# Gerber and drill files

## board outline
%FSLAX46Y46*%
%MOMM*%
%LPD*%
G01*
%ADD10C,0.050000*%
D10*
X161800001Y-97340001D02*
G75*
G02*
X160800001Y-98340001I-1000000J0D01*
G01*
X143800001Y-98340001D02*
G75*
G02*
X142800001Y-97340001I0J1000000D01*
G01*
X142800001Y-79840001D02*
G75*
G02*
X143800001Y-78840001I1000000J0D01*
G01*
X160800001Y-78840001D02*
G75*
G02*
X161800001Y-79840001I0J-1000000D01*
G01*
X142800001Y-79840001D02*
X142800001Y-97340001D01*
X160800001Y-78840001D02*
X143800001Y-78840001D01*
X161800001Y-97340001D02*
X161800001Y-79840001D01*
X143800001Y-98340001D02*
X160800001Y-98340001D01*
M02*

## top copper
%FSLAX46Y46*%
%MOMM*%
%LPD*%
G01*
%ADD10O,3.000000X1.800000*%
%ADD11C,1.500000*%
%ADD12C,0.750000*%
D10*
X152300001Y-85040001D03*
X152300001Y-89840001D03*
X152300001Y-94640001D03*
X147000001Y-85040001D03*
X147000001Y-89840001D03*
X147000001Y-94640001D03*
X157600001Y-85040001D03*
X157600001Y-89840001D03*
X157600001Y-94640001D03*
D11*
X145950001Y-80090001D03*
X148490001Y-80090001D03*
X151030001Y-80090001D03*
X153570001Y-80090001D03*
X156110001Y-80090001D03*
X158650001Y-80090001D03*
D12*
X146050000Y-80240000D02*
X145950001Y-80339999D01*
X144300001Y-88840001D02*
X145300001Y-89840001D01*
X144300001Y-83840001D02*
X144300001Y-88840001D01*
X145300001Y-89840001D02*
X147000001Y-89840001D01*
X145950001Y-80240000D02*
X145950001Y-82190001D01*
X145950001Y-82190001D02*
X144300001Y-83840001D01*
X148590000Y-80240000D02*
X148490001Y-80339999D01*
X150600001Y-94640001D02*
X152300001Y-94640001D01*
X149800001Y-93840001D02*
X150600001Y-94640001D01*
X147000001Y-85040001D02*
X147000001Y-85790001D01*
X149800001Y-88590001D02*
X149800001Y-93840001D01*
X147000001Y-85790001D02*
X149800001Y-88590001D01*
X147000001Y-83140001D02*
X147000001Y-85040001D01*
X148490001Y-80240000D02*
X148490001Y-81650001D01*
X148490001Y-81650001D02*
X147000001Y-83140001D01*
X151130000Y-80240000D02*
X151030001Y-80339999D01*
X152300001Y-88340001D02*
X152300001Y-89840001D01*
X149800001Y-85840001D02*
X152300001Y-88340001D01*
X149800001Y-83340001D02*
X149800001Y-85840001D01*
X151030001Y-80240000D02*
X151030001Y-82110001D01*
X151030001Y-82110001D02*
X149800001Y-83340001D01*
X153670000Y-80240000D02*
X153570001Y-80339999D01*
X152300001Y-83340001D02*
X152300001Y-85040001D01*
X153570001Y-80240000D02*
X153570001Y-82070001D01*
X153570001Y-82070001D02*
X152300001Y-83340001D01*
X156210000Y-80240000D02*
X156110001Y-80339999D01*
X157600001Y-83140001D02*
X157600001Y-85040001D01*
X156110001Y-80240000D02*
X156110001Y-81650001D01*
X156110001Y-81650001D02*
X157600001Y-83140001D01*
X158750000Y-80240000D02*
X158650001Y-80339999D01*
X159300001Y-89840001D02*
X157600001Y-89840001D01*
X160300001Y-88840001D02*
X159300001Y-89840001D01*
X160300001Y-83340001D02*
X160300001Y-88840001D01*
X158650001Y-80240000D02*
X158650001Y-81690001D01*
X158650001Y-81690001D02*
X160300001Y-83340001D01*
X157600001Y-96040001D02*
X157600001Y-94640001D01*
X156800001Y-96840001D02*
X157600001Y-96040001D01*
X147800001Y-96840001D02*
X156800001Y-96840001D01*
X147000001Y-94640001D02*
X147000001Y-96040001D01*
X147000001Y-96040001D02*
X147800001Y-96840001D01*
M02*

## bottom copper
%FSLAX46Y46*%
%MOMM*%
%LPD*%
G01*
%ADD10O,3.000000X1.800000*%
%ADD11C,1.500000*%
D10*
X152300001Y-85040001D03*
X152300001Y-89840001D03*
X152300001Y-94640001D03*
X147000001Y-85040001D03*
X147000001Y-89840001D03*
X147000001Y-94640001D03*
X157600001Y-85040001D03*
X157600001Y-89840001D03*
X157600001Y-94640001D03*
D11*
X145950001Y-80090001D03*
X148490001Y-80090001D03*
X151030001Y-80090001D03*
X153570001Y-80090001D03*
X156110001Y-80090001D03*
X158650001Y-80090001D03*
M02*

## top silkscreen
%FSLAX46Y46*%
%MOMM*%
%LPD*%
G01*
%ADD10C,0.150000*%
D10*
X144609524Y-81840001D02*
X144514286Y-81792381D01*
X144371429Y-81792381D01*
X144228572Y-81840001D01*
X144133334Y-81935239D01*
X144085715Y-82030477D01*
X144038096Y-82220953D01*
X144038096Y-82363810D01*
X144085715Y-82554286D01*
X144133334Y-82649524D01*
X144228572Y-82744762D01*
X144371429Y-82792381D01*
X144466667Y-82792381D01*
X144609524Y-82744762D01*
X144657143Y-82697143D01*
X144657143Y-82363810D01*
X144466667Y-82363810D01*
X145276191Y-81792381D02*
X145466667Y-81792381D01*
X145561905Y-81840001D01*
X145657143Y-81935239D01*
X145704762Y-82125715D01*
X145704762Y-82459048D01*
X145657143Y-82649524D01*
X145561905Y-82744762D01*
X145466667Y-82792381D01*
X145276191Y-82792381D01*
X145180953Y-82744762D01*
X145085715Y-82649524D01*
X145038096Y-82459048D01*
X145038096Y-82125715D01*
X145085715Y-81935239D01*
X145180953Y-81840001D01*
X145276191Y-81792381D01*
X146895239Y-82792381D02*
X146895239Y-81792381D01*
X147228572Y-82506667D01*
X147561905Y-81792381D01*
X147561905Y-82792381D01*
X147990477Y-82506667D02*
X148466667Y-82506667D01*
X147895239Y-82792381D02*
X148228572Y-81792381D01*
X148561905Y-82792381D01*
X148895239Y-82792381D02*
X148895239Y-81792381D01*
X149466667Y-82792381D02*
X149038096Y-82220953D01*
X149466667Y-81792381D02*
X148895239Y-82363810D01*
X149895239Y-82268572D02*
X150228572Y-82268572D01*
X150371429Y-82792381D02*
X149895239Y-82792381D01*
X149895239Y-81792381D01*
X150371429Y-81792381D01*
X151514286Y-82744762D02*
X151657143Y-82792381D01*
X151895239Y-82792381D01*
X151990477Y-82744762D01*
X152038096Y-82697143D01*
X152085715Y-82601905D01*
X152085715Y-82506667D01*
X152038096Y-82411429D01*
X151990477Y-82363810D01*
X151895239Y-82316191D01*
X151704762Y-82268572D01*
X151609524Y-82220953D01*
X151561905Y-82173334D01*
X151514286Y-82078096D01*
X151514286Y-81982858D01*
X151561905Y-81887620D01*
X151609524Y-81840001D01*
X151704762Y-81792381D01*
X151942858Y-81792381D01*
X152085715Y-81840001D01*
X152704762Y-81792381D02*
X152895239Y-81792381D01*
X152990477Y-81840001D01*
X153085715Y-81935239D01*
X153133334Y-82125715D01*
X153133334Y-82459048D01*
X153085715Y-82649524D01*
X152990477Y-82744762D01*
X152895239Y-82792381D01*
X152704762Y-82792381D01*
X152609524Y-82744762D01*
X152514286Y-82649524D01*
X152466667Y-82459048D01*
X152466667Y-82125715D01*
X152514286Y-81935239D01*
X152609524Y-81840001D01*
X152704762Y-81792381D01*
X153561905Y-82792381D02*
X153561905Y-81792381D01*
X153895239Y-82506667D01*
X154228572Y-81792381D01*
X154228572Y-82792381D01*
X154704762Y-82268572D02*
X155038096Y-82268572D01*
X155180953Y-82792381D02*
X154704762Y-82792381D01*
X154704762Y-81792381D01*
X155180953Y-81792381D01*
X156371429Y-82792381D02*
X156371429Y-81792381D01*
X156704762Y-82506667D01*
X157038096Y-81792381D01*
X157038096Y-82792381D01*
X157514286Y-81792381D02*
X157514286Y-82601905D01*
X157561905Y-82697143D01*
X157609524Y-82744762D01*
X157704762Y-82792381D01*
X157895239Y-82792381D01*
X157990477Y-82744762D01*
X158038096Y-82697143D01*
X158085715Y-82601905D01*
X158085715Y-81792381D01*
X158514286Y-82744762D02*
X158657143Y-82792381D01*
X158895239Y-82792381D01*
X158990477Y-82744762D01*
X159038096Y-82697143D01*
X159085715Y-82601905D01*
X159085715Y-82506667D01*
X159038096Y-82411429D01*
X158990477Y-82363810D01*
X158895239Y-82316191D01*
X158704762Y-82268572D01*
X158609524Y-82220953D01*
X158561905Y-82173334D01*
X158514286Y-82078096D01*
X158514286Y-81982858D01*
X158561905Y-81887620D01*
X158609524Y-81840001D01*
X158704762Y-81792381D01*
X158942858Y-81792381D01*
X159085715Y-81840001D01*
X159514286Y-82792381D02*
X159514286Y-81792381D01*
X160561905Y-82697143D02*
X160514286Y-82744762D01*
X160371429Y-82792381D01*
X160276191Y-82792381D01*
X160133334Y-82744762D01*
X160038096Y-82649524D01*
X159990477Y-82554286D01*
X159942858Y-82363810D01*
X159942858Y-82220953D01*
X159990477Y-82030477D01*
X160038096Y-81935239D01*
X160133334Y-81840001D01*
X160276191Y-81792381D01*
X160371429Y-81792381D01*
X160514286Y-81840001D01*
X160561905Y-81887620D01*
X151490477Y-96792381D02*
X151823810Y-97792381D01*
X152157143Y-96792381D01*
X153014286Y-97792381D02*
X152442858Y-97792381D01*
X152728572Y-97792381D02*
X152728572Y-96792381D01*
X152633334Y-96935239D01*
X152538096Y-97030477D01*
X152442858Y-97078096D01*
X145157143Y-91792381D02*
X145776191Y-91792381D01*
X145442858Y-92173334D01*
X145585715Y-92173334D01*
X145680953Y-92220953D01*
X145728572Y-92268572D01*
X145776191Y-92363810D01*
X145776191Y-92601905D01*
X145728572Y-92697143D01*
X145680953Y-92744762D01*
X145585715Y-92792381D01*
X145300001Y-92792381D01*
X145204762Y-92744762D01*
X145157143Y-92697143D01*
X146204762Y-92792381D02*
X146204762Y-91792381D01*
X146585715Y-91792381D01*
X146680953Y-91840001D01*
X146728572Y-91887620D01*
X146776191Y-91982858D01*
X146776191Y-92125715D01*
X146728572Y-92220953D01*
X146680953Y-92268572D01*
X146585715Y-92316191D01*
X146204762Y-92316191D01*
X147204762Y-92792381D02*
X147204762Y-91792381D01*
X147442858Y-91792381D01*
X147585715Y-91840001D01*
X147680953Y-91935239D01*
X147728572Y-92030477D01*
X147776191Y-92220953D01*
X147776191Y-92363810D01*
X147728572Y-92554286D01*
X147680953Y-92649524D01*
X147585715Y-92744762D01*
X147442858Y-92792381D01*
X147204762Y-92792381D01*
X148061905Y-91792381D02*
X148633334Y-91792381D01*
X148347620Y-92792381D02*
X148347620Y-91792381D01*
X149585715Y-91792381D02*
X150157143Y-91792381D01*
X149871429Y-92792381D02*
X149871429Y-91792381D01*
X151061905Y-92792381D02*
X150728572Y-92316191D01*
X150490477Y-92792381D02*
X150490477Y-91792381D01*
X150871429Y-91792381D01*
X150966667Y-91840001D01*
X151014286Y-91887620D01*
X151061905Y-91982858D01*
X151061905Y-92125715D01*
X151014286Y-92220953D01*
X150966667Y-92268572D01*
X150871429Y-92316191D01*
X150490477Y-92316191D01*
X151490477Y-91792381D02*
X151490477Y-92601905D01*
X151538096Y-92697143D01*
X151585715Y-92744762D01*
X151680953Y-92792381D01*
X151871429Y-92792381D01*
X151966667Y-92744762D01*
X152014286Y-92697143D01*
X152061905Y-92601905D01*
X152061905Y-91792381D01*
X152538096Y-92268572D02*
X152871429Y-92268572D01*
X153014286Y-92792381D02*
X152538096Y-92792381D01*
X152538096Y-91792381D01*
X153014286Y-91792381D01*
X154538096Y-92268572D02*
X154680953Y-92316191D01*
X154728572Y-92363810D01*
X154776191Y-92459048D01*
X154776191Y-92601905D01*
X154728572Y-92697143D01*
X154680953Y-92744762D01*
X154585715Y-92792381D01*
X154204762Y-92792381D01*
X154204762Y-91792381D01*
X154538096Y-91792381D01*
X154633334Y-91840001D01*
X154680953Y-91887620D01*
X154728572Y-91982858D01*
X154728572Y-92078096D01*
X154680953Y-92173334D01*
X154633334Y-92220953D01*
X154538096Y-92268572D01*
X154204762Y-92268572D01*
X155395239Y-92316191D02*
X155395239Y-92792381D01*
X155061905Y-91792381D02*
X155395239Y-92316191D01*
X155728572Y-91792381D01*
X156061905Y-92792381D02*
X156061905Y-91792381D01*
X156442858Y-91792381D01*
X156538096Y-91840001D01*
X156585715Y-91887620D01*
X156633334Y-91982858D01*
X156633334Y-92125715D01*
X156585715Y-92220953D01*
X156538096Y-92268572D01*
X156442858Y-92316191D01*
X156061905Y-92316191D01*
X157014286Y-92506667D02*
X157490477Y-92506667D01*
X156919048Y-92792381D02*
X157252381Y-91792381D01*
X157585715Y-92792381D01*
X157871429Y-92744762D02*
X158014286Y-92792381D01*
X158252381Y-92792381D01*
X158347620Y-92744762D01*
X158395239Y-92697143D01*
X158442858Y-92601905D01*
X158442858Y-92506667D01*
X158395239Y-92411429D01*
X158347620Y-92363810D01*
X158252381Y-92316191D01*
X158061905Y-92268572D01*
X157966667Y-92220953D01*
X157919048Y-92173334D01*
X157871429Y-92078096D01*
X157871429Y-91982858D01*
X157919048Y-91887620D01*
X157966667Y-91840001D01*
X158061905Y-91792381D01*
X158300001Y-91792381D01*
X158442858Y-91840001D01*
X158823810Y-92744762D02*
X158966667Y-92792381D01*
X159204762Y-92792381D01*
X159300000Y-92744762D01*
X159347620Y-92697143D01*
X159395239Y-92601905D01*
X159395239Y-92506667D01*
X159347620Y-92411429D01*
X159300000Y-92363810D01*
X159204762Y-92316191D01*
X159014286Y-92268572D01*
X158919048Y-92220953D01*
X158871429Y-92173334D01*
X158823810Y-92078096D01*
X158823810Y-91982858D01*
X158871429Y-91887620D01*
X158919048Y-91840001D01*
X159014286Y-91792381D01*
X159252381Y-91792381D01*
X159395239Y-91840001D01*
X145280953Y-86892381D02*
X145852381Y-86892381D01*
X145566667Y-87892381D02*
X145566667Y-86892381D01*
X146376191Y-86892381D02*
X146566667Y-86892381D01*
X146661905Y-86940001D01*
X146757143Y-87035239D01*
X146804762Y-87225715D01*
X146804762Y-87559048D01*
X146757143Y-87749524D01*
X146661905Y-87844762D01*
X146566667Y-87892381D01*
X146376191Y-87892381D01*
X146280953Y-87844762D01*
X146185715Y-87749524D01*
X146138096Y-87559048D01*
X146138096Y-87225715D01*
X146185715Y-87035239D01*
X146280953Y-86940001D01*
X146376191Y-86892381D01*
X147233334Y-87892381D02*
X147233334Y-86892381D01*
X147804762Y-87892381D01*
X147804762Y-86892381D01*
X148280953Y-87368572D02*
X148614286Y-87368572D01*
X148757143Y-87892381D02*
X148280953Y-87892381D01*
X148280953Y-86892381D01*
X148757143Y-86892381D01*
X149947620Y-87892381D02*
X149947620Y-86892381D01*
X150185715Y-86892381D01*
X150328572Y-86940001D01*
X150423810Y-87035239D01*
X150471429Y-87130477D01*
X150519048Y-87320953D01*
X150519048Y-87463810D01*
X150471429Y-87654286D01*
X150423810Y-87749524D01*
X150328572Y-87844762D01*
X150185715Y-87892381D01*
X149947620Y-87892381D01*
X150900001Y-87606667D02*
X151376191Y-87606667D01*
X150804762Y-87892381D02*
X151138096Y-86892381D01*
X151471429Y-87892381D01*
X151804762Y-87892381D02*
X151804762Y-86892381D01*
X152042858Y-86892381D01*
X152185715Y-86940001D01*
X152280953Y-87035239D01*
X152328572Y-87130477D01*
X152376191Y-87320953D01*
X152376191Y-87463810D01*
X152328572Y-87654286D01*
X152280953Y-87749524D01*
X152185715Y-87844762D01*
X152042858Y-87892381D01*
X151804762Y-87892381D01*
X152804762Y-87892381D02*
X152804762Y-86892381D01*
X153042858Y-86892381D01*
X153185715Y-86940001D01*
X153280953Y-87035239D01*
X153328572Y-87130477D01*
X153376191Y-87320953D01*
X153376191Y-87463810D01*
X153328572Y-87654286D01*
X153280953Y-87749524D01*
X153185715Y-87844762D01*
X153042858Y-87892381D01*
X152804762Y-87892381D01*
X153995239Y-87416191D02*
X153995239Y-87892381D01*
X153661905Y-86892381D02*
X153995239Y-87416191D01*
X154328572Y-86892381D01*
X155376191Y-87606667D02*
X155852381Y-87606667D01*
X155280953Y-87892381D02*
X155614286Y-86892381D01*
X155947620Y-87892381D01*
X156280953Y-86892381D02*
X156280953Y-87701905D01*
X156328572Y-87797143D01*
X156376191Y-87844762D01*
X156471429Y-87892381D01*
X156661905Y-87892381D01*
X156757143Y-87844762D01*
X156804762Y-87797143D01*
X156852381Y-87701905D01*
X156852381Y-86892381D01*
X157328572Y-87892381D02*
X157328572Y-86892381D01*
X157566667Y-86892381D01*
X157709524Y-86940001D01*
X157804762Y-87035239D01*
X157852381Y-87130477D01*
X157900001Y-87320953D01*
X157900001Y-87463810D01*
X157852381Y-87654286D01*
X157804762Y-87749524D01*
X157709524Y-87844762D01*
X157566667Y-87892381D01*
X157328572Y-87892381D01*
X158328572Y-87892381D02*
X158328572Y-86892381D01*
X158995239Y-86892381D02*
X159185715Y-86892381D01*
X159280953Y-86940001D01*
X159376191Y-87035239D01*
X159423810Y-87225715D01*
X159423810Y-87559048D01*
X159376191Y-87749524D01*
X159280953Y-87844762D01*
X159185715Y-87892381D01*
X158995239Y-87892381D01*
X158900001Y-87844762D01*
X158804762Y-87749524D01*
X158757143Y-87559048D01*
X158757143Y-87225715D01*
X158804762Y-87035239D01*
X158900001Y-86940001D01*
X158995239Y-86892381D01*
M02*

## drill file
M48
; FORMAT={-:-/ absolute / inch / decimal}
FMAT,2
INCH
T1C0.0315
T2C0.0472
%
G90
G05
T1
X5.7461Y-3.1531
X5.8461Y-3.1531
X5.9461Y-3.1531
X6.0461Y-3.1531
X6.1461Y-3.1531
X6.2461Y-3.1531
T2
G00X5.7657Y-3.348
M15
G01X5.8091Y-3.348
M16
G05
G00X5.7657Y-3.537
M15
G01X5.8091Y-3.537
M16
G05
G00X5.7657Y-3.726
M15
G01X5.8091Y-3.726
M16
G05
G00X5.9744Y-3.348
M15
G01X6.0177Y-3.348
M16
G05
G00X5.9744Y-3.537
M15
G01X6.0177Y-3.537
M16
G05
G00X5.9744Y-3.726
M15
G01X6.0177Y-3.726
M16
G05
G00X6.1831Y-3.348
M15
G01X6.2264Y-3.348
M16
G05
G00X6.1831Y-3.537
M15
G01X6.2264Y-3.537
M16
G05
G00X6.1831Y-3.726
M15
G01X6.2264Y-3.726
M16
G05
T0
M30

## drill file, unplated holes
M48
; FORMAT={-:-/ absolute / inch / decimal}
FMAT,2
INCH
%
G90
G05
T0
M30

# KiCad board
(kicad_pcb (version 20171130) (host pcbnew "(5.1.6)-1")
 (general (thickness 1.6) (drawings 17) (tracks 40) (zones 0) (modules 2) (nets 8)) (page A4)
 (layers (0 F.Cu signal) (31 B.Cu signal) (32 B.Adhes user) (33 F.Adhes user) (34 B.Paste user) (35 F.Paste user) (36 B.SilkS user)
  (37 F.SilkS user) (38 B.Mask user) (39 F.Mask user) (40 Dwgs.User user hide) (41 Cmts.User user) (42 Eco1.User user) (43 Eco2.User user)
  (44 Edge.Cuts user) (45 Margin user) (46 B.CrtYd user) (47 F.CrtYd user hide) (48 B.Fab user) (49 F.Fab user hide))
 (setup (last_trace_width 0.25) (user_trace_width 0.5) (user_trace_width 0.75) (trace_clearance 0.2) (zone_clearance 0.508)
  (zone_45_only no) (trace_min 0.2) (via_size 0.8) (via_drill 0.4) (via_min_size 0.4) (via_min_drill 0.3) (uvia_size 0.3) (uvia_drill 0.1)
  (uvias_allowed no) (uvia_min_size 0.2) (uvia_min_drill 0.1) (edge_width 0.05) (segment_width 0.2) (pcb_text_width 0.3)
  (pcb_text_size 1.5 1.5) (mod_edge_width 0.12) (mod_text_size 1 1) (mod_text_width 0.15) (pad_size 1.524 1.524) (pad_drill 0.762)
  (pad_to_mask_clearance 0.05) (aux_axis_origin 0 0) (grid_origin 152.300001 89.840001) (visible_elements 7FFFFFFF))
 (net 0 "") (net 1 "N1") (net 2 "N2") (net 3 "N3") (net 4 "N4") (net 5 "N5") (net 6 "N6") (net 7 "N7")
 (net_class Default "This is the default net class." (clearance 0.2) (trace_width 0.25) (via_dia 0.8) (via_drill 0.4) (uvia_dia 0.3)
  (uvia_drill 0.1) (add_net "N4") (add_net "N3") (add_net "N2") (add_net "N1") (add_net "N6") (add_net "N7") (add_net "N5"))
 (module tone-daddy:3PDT (layer F.Cu) (at 152.300001 89.840001)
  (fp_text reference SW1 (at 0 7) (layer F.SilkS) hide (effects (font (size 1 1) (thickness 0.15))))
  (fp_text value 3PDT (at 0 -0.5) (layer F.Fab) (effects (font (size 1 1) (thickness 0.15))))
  (pad 4 thru_hole oval (at 0 -4.8) (size 3 1.8) (drill oval 2.3 1.2) (layers *.Cu *.Mask) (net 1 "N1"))
  (pad 5 thru_hole oval (at 0 0) (size 3 1.8) (drill oval 2.3 1.2) (layers *.Cu *.Mask) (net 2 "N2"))
  (pad 6 thru_hole oval (at 0 4.8) (size 3 1.8) (drill oval 2.3 1.2) (layers *.Cu *.Mask) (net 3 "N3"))
  (pad 1 thru_hole oval (at -5.3 -4.8) (size 3 1.8) (drill oval 2.3 1.2) (layers *.Cu *.Mask) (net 3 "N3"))
  (pad 2 thru_hole oval (at -5.3 0) (size 3 1.8) (drill oval 2.3 1.2) (layers *.Cu *.Mask) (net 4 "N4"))
  (pad 3 thru_hole oval (at -5.3 4.8) (size 3 1.8) (drill oval 2.3 1.2) (layers *.Cu *.Mask) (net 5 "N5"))
  (pad 7 thru_hole oval (at 5.3 -4.8) (size 3 1.8) (drill oval 2.3 1.2) (layers *.Cu *.Mask) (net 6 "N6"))
  (pad 8 thru_hole oval (at 5.3 0) (size 3 1.8) (drill oval 2.3 1.2) (layers *.Cu *.Mask) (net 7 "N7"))
  (pad 9 thru_hole oval (at 5.3 4.8) (size 3 1.8) (drill oval 2.3 1.2) (layers *.Cu *.Mask) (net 5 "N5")))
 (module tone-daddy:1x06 (layer F.Cu) (at 152.300001 80.090001)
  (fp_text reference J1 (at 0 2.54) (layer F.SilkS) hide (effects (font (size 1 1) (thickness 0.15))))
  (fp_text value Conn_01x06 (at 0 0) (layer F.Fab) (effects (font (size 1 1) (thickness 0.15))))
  (pad 1 thru_hole circle (at -6.35 0) (size 1.5 1.5) (drill 0.8) (layers *.Cu *.Mask) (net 4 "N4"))
  (pad 2 thru_hole circle (at -3.81 0) (size 1.5 1.5) (drill 0.8) (layers *.Cu *.Mask) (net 3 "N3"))
  (pad 3 thru_hole circle (at -1.27 0) (size 1.5 1.5) (drill 0.8) (layers *.Cu *.Mask) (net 2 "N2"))
  (pad 4 thru_hole circle (at 1.27 0) (size 1.5 1.5) (drill 0.8) (layers *.Cu *.Mask) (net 1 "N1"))
  (pad 5 thru_hole circle (at 3.81 0) (size 1.5 1.5) (drill 0.8) (layers *.Cu *.Mask) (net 6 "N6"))
  (pad 6 thru_hole circle (at 6.35 0) (size 1.5 1.5) (drill 0.8) (layers *.Cu *.Mask) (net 7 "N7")))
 (gr_arc (start 160.800001 97.340001) (end 160.800001 98.340001) (angle -90) (layer Edge.Cuts) (width 0.05))
 (gr_arc (start 143.800001 97.340001) (end 142.800001 97.340001) (angle -90) (layer Edge.Cuts) (width 0.05))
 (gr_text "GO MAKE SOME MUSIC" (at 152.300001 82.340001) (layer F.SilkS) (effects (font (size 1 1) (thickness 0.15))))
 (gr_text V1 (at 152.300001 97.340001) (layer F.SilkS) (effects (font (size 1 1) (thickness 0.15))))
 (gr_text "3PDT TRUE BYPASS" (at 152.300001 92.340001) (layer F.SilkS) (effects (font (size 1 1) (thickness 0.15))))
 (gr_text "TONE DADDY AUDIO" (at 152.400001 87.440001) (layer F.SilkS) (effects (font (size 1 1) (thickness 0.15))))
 (gr_arc (start 143.800001 79.840001) (end 143.800001 78.840001) (angle -90) (layer Edge.Cuts) (width 0.05))
 (gr_arc (start 160.800001 79.840001) (end 161.800001 79.840001) (angle -90) (layer Edge.Cuts) (width 0.05))
 (gr_line (start 142.800001 79.840001) (end 142.800001 97.340001) (layer Edge.Cuts) (width 0.05))
 (gr_line (start 160.800001 78.840001) (end 143.800001 78.840001) (layer Edge.Cuts) (width 0.05))
 (gr_line (start 161.800001 97.340001) (end 161.800001 79.840001) (layer Edge.Cuts) (width 0.05))
 (gr_line (start 143.800001 98.340001) (end 160.800001 98.340001) (layer Edge.Cuts) (width 0.05))
 (segment (start 146.05 80.24) (end 145.950001 80.339999) (width 0.75) (layer F.Cu) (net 4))
 (segment (start 144.300001 88.840001) (end 145.300001 89.840001) (width 0.75) (layer F.Cu) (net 4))
 (segment (start 144.300001 83.840001) (end 144.300001 88.840001) (width 0.75) (layer F.Cu) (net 4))
 (segment (start 145.300001 89.840001) (end 147.000001 89.840001) (width 0.75) (layer F.Cu) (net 4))
 (segment (start 145.950001 80.24) (end 145.950001 82.190001) (width 0.75) (layer F.Cu) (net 4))
 (segment (start 145.950001 82.190001) (end 144.300001 83.840001) (width 0.75) (layer F.Cu) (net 4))
 (segment (start 148.59 80.24) (end 148.490001 80.339999) (width 0.75) (layer F.Cu) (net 3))
 (segment (start 150.600001 94.640001) (end 152.300001 94.640001) (width 0.75) (layer F.Cu) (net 3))
 (segment (start 149.800001 93.840001) (end 150.600001 94.640001) (width 0.75) (layer F.Cu) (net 3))
 (segment (start 147.000001 85.040001) (end 147.000001 85.790001) (width 0.75) (layer F.Cu) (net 3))
 (segment (start 149.800001 88.590001) (end 149.800001 93.840001) (width 0.75) (layer F.Cu) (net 3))
 (segment (start 147.000001 85.790001) (end 149.800001 88.590001) (width 0.75) (layer F.Cu) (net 3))
 (segment (start 147.000001 83.140001) (end 147.000001 85.040001) (width 0.75) (layer F.Cu) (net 3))
 (segment (start 148.490001 80.24) (end 148.490001 81.650001) (width 0.75) (layer F.Cu) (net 3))
 (segment (start 148.490001 81.650001) (end 147.000001 83.140001) (width 0.75) (layer F.Cu) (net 3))
 (segment (start 151.13 80.24) (end 151.030001 80.339999) (width 0.75) (layer F.Cu) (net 2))
 (segment (start 152.300001 88.340001) (end 152.300001 89.840001) (width 0.75) (layer F.Cu) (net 2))
 (segment (start 149.800001 85.840001) (end 152.300001 88.340001) (width 0.75) (layer F.Cu) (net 2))
 (segment (start 149.800001 83.340001) (end 149.800001 85.840001) (width 0.75) (layer F.Cu) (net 2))
 (segment (start 151.030001 80.24) (end 151.030001 82.110001) (width 0.75) (layer F.Cu) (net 2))
 (segment (start 151.030001 82.110001) (end 149.800001 83.340001) (width 0.75) (layer F.Cu) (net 2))
 (segment (start 153.67 80.24) (end 153.570001 80.339999) (width 0.75) (layer F.Cu) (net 1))
 (segment (start 152.300001 83.340001) (end 152.300001 85.040001) (width 0.75) (layer F.Cu) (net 1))
 (segment (start 153.570001 80.24) (end 153.570001 82.070001) (width 0.75) (layer F.Cu) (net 1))
 (segment (start 153.570001 82.070001) (end 152.300001 83.340001) (width 0.75) (layer F.Cu) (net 1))
 (segment (start 156.21 80.24) (end 156.110001 80.339999) (width 0.75) (layer F.Cu) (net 6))
 (segment (start 157.600001 83.140001) (end 157.600001 85.040001) (width 0.75) (layer F.Cu) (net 6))
 (segment (start 156.110001 80.24) (end 156.110001 81.650001) (width 0.75) (layer F.Cu) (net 6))
 (segment (start 156.110001 81.650001) (end 157.600001 83.140001) (width 0.75) (layer F.Cu) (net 6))
 (segment (start 158.75 80.24) (end 158.650001 80.339999) (width 0.75) (layer F.Cu) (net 7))
 (segment (start 159.300001 89.840001) (end 157.600001 89.840001) (width 0.75) (layer F.Cu) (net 7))
 (segment (start 160.300001 88.840001) (end 159.300001 89.840001) (width 0.75) (layer F.Cu) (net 7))
 (segment (start 160.300001 83.340001) (end 160.300001 88.840001) (width 0.75) (layer F.Cu) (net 7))
 (segment (start 158.650001 80.24) (end 158.650001 81.690001) (width 0.75) (layer F.Cu) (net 7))
 (segment (start 158.650001 81.690001) (end 160.300001 83.340001) (width 0.75) (layer F.Cu) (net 7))
 (segment (start 157.600001 96.040001) (end 157.600001 94.640001) (width 0.75) (layer F.Cu) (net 5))
 (segment (start 156.800001 96.840001) (end 157.600001 96.040001) (width 0.75) (layer F.Cu) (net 5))
 (segment (start 147.800001 96.840001) (end 156.800001 96.840001) (width 0.75) (layer F.Cu) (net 5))
 (segment (start 147.000001 94.640001) (end 147.000001 96.040001) (width 0.75) (layer F.Cu) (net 5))
 (segment (start 147.000001 96.040001) (end 147.800001 96.840001) (width 0.75) (layer F.Cu) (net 5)))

